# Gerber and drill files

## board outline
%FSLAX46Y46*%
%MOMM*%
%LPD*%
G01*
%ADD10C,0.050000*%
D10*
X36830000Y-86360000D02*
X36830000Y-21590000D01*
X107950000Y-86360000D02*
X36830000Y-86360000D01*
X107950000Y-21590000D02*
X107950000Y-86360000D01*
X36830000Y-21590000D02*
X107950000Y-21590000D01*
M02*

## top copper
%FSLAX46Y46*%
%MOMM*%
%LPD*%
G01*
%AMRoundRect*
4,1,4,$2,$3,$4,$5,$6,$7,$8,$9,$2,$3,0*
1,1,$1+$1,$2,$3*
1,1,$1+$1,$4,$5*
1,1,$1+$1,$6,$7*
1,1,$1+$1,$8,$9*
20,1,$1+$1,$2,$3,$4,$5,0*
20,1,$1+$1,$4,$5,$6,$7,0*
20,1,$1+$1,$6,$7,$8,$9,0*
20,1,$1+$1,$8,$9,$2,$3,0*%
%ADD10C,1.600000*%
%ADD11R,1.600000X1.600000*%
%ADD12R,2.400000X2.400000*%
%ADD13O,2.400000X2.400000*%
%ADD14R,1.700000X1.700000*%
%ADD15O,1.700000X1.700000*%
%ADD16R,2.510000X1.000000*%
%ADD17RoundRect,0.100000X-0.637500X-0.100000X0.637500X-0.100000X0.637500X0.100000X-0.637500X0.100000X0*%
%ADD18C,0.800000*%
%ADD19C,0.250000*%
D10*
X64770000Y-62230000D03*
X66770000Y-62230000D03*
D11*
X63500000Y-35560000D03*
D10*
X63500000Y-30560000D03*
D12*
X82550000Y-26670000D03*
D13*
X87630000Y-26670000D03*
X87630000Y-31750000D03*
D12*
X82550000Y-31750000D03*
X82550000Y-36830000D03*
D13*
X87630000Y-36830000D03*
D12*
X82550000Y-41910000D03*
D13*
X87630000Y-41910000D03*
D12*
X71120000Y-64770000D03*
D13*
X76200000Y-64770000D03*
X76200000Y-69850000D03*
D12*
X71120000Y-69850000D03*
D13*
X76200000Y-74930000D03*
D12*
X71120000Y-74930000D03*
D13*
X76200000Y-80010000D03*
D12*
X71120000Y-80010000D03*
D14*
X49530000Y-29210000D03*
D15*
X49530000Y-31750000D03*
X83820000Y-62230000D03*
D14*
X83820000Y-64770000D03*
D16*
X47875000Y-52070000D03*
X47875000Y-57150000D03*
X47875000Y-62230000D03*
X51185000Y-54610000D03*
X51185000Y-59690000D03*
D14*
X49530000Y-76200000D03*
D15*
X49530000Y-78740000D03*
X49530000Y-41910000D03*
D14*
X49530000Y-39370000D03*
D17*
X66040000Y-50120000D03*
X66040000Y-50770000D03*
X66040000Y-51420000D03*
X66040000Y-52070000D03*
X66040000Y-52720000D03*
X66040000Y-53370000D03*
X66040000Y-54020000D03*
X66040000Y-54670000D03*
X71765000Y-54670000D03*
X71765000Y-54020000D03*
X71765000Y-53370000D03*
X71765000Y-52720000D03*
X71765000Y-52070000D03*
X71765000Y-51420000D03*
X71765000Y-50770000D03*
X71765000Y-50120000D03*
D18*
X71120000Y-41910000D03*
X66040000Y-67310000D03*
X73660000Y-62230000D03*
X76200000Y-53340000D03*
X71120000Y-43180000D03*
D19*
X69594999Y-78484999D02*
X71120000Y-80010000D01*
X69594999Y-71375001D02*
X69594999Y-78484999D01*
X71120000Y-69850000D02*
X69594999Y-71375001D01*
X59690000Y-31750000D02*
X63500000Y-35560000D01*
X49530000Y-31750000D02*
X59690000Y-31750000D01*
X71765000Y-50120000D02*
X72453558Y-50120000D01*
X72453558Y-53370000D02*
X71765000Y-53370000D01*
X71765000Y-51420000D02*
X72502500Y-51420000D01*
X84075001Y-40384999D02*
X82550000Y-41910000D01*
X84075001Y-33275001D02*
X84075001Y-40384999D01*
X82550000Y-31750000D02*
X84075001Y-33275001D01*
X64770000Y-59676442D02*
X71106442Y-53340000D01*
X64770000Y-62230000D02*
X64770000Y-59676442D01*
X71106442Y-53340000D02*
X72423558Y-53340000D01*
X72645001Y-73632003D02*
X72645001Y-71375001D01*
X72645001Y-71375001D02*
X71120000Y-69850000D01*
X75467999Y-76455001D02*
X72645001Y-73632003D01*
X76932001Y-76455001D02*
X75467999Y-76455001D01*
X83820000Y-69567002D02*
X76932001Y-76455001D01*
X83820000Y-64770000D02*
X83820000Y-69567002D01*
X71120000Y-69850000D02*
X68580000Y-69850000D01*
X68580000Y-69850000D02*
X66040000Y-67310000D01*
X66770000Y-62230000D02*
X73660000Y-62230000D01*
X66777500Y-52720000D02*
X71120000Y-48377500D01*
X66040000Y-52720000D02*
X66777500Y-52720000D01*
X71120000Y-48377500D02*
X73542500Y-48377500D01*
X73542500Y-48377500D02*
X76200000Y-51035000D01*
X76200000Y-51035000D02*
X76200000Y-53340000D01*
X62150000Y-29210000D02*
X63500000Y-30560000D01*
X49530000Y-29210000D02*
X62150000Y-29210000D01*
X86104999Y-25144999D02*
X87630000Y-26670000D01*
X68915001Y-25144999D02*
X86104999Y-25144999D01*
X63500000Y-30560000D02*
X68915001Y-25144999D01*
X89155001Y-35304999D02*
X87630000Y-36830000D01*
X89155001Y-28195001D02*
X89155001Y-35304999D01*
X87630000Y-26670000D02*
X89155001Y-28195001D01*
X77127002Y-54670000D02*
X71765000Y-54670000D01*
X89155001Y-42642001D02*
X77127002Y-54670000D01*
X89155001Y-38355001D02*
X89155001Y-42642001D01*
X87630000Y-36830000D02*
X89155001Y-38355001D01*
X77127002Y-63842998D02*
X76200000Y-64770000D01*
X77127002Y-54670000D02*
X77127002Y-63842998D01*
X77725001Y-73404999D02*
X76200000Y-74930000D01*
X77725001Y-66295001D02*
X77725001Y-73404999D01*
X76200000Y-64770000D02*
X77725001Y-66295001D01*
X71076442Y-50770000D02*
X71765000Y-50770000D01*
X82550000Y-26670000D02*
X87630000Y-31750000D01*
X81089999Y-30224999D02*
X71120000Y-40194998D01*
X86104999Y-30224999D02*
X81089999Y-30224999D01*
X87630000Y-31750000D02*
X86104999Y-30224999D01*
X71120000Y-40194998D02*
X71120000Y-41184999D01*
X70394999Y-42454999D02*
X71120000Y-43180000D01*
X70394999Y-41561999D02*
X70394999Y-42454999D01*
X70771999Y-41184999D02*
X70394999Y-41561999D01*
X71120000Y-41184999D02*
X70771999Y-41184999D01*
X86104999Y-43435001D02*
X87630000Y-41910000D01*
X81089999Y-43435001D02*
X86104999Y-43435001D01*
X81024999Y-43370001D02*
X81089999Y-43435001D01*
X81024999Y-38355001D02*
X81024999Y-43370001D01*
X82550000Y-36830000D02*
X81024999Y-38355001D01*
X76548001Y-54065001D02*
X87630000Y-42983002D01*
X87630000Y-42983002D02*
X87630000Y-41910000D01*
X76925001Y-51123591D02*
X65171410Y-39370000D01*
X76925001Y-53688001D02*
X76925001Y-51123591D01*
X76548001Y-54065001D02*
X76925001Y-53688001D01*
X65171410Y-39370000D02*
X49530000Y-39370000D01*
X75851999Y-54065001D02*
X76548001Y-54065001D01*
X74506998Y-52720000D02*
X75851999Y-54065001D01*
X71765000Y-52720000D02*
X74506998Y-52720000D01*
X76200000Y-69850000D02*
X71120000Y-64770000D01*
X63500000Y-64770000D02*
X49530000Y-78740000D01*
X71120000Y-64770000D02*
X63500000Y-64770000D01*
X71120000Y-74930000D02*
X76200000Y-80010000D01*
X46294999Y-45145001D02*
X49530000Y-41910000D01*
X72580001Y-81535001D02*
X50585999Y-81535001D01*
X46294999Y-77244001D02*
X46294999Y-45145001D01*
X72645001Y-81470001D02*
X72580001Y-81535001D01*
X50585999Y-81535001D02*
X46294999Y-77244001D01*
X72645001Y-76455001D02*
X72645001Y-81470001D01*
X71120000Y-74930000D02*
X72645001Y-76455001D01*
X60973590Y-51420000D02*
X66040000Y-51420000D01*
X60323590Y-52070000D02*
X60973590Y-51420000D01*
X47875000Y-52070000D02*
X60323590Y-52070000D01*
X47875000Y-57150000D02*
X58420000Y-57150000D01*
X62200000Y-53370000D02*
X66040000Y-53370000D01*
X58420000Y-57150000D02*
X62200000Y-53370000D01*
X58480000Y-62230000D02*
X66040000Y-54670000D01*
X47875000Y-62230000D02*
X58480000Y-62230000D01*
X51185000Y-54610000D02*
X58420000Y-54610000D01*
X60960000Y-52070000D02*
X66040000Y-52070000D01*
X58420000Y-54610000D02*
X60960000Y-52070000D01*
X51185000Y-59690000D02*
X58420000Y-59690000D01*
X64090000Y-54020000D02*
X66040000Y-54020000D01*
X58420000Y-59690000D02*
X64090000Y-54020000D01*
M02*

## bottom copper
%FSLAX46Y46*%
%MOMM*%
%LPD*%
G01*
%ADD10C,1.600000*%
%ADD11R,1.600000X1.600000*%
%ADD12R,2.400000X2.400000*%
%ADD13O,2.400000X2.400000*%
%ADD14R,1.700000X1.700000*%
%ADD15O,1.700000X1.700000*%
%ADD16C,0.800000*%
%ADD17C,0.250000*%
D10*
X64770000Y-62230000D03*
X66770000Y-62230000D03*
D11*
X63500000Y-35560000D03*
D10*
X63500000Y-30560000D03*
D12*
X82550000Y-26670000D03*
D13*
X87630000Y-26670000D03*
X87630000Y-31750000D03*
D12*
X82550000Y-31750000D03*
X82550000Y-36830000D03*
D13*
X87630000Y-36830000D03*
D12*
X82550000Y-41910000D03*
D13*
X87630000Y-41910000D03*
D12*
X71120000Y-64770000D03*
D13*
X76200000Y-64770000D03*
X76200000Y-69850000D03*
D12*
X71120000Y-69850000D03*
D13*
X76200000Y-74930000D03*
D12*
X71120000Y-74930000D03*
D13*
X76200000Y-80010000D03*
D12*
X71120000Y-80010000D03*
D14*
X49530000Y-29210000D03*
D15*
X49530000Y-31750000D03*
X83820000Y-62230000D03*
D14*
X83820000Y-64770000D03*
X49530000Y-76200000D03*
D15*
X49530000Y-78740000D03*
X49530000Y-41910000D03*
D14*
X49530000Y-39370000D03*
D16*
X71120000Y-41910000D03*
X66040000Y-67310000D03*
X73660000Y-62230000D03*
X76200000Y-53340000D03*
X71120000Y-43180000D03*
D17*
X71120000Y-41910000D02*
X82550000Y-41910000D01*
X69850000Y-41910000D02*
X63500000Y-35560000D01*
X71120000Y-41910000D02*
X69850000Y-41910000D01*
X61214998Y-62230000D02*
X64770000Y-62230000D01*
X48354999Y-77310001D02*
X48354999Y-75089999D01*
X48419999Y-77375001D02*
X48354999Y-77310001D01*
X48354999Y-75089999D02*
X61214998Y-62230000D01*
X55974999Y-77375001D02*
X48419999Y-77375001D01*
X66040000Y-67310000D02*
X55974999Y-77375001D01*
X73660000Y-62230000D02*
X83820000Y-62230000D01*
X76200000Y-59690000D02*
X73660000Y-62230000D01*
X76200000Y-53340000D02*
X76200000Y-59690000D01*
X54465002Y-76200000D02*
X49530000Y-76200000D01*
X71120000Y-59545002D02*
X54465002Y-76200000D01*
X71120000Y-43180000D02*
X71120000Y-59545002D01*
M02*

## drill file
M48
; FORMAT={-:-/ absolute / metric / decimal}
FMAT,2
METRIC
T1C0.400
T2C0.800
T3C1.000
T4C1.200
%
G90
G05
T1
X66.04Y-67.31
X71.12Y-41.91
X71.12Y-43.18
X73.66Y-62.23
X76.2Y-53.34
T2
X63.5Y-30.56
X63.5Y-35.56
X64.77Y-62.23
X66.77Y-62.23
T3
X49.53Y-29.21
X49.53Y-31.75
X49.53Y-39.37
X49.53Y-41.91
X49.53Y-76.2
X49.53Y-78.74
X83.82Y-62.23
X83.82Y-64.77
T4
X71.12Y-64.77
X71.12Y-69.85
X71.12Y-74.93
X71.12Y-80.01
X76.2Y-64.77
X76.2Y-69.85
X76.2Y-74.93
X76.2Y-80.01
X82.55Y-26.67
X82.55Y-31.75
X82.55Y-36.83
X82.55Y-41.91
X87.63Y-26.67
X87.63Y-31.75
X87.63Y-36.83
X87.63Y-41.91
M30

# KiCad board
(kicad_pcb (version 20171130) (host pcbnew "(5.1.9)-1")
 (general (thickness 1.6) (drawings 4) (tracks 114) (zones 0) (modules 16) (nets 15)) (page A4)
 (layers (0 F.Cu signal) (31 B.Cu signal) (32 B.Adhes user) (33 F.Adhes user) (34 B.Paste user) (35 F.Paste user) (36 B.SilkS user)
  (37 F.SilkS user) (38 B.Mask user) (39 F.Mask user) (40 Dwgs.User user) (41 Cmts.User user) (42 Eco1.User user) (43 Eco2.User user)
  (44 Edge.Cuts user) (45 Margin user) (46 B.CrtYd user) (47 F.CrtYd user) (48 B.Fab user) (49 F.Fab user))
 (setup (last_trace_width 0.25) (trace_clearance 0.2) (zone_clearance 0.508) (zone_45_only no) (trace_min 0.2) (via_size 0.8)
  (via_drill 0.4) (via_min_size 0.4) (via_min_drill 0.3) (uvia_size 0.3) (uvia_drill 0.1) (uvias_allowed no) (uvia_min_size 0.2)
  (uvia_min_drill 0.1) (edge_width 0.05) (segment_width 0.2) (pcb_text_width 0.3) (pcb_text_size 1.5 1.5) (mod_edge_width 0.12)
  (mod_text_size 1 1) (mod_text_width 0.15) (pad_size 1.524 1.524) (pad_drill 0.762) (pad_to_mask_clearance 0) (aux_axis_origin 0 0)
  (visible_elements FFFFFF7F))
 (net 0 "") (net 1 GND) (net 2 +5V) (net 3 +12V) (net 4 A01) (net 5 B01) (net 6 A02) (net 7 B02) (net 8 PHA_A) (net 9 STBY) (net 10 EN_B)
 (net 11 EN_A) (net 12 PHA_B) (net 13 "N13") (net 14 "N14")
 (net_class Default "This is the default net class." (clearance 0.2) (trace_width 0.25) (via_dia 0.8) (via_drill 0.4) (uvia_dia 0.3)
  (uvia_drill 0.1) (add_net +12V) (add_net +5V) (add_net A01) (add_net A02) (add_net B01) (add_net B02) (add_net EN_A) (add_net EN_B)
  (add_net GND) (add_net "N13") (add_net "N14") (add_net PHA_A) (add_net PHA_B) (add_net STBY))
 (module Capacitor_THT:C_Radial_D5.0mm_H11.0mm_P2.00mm (layer F.Cu) (at 64.77 62.23)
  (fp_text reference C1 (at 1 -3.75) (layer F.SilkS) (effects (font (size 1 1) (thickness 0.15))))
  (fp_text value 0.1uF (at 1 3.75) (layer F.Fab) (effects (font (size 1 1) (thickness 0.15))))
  (pad 1 thru_hole circle (at 0 0) (size 1.6 1.6) (drill 0.8) (layers *.Cu *.Mask) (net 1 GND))
  (pad 2 thru_hole circle (at 2 0) (size 1.6 1.6) (drill 0.8) (layers *.Cu *.Mask) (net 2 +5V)))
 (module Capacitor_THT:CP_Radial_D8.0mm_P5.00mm (layer F.Cu) (at 63.5 35.56 90)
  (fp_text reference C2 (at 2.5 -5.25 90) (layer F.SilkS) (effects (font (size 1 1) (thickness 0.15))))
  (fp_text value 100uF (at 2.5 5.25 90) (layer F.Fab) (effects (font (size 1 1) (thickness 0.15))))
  (pad 1 thru_hole rect (at 0 0 90) (size 1.6 1.6) (drill 0.8) (layers *.Cu *.Mask) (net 1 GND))
  (pad 2 thru_hole circle (at 5 0 90) (size 1.6 1.6) (drill 0.8) (layers *.Cu *.Mask) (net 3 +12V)))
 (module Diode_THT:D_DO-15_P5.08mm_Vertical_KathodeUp (layer F.Cu) (at 82.55 26.67)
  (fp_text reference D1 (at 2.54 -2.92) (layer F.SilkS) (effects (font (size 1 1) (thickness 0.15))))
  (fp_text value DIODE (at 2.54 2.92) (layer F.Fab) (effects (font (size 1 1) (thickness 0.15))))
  (pad 1 thru_hole rect (at 0 0) (size 2.4 2.4) (drill 1.2) (layers *.Cu *.Mask) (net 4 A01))
  (pad 2 thru_hole oval (at 5.08 0) (size 2.4 2.4) (drill 1.2) (layers *.Cu *.Mask) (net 3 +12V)))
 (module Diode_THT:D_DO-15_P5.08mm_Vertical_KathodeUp (layer F.Cu) (at 82.55 31.75)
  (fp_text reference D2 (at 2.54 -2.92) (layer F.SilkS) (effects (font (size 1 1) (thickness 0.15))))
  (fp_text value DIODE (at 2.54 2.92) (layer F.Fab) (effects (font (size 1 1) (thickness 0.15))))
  (pad 2 thru_hole oval (at 5.08 0) (size 2.4 2.4) (drill 1.2) (layers *.Cu *.Mask) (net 4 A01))
  (pad 1 thru_hole rect (at 0 0) (size 2.4 2.4) (drill 1.2) (layers *.Cu *.Mask) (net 1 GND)))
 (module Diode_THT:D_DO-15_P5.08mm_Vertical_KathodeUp (layer F.Cu) (at 82.55 36.83)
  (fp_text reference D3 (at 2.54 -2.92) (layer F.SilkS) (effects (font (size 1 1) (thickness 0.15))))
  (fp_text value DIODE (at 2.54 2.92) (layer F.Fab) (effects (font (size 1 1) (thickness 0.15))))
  (pad 1 thru_hole rect (at 0 0) (size 2.4 2.4) (drill 1.2) (layers *.Cu *.Mask) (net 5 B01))
  (pad 2 thru_hole oval (at 5.08 0) (size 2.4 2.4) (drill 1.2) (layers *.Cu *.Mask) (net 3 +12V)))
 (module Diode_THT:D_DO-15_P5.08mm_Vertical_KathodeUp (layer F.Cu) (at 82.55 41.91)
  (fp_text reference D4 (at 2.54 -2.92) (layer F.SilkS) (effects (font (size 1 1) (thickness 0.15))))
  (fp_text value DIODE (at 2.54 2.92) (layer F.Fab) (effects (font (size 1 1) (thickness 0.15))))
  (pad 1 thru_hole rect (at 0 0) (size 2.4 2.4) (drill 1.2) (layers *.Cu *.Mask) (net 1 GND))
  (pad 2 thru_hole oval (at 5.08 0) (size 2.4 2.4) (drill 1.2) (layers *.Cu *.Mask) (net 5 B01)))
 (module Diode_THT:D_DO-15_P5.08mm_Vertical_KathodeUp (layer F.Cu) (at 71.12 64.77)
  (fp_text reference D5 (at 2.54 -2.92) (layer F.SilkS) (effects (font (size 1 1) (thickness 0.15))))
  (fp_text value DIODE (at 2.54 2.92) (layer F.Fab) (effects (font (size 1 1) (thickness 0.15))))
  (pad 1 thru_hole rect (at 0 0) (size 2.4 2.4) (drill 1.2) (layers *.Cu *.Mask) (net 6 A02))
  (pad 2 thru_hole oval (at 5.08 0) (size 2.4 2.4) (drill 1.2) (layers *.Cu *.Mask) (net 3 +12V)))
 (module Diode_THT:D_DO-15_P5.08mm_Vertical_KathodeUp (layer F.Cu) (at 71.12 69.85)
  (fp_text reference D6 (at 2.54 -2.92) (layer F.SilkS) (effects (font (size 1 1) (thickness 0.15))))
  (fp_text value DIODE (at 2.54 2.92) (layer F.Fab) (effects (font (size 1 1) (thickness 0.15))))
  (pad 2 thru_hole oval (at 5.08 0) (size 2.4 2.4) (drill 1.2) (layers *.Cu *.Mask) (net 6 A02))
  (pad 1 thru_hole rect (at 0 0) (size 2.4 2.4) (drill 1.2) (layers *.Cu *.Mask) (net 1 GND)))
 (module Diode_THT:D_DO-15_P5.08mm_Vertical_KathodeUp (layer F.Cu) (at 71.12 74.93)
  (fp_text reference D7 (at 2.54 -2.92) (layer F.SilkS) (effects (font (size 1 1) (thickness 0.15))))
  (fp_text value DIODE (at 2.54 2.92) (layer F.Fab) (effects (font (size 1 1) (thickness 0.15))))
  (pad 2 thru_hole oval (at 5.08 0) (size 2.4 2.4) (drill 1.2) (layers *.Cu *.Mask) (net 3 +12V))
  (pad 1 thru_hole rect (at 0 0) (size 2.4 2.4) (drill 1.2) (layers *.Cu *.Mask) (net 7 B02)))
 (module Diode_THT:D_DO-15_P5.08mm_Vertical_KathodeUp (layer F.Cu) (at 71.12 80.01)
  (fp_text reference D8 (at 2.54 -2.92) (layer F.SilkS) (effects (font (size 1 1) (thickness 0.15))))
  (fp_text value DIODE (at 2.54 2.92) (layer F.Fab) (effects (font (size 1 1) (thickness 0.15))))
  (pad 2 thru_hole oval (at 5.08 0) (size 2.4 2.4) (drill 1.2) (layers *.Cu *.Mask) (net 7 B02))
  (pad 1 thru_hole rect (at 0 0) (size 2.4 2.4) (drill 1.2) (layers *.Cu *.Mask) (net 1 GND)))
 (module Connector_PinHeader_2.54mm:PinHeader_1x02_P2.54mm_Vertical (layer F.Cu) (at 49.53 29.21)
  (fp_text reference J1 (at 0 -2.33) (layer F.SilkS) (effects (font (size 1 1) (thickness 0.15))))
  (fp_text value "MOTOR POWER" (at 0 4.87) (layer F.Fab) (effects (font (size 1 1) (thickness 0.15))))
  (pad 1 thru_hole rect (at 0 0) (size 1.7 1.7) (drill 1) (layers *.Cu *.Mask) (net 3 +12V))
  (pad 2 thru_hole oval (at 0 2.54) (size 1.7 1.7) (drill 1) (layers *.Cu *.Mask) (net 1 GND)))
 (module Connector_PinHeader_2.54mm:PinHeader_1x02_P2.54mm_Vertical (layer F.Cu) (at 83.82 64.77 180)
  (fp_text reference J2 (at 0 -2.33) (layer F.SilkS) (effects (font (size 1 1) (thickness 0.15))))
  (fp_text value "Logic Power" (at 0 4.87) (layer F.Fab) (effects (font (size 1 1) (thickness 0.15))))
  (pad 2 thru_hole oval (at 0 2.54 180) (size 1.7 1.7) (drill 1) (layers *.Cu *.Mask) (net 2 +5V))
  (pad 1 thru_hole rect (at 0 0 180) (size 1.7 1.7) (drill 1) (layers *.Cu *.Mask) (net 1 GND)))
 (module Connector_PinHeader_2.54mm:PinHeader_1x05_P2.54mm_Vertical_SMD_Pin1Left (layer F.Cu) (at 49.53 57.15)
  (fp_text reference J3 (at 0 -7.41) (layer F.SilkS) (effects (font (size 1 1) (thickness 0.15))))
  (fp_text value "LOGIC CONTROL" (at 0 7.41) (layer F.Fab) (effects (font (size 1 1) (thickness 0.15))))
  (pad 1 smd rect (at -1.655 -5.08) (size 2.51 1) (layers F.Cu F.Paste F.Mask) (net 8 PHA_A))
  (pad 3 smd rect (at -1.655 0) (size 2.51 1) (layers F.Cu F.Paste F.Mask) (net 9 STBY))
  (pad 5 smd rect (at -1.655 5.08) (size 2.51 1) (layers F.Cu F.Paste F.Mask) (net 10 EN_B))
  (pad 2 smd rect (at 1.655 -2.54) (size 2.51 1) (layers F.Cu F.Paste F.Mask) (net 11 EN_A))
  (pad 4 smd rect (at 1.655 2.54) (size 2.51 1) (layers F.Cu F.Paste F.Mask) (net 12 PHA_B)))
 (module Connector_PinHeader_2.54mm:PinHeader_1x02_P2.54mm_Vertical (layer F.Cu) (at 49.53 76.2)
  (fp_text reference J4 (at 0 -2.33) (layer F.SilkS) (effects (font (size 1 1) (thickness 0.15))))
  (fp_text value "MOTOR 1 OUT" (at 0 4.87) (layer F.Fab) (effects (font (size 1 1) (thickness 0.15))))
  (pad 1 thru_hole rect (at 0 0) (size 1.7 1.7) (drill 1) (layers *.Cu *.Mask) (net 4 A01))
  (pad 2 thru_hole oval (at 0 2.54) (size 1.7 1.7) (drill 1) (layers *.Cu *.Mask) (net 6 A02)))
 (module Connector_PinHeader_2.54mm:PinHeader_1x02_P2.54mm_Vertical (layer F.Cu) (at 49.53 39.37)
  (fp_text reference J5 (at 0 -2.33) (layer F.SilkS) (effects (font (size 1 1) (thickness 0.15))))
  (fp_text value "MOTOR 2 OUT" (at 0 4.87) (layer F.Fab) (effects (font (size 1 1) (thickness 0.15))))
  (pad 2 thru_hole oval (at 0 2.54) (size 1.7 1.7) (drill 1) (layers *.Cu *.Mask) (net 7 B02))
  (pad 1 thru_hole rect (at 0 0) (size 1.7 1.7) (drill 1) (layers *.Cu *.Mask) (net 5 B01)))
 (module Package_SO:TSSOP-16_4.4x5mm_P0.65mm (layer F.Cu) (at 68.9025 52.395)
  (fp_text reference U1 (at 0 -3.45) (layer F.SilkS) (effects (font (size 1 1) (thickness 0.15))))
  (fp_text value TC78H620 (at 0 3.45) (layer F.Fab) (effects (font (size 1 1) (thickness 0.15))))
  (pad 1 smd roundrect (at -2.8625 -2.275) (size 1.475 0.4) (layers F.Cu F.Paste F.Mask) (roundrect_rratio 0.25) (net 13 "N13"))
  (pad 2 smd roundrect (at -2.8625 -1.625) (size 1.475 0.4) (layers F.Cu F.Paste F.Mask) (roundrect_rratio 0.25) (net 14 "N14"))
  (pad 3 smd roundrect (at -2.8625 -0.975) (size 1.475 0.4) (layers F.Cu F.Paste F.Mask) (roundrect_rratio 0.25) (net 8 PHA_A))
  (pad 4 smd roundrect (at -2.8625 -0.325) (size 1.475 0.4) (layers F.Cu F.Paste F.Mask) (roundrect_rratio 0.25) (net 11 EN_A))
  (pad 5 smd roundrect (at -2.8625 0.325) (size 1.475 0.4) (layers F.Cu F.Paste F.Mask) (roundrect_rratio 0.25) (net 2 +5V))
  (pad 6 smd roundrect (at -2.8625 0.975) (size 1.475 0.4) (layers F.Cu F.Paste F.Mask) (roundrect_rratio 0.25) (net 9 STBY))
  (pad 7 smd roundrect (at -2.8625 1.625) (size 1.475 0.4) (layers F.Cu F.Paste F.Mask) (roundrect_rratio 0.25) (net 12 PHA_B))
  (pad 8 smd roundrect (at -2.8625 2.275) (size 1.475 0.4) (layers F.Cu F.Paste F.Mask) (roundrect_rratio 0.25) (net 10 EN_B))
  (pad 9 smd roundrect (at 2.8625 2.275) (size 1.475 0.4) (layers F.Cu F.Paste F.Mask) (roundrect_rratio 0.25) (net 3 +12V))
  (pad 10 smd roundrect (at 2.8625 1.625) (size 1.475 0.4) (layers F.Cu F.Paste F.Mask) (roundrect_rratio 0.25) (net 7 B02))
  (pad 11 smd roundrect (at 2.8625 0.975) (size 1.475 0.4) (layers F.Cu F.Paste F.Mask) (roundrect_rratio 0.25) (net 1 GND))
  (pad 12 smd roundrect (at 2.8625 0.325) (size 1.475 0.4) (layers F.Cu F.Paste F.Mask) (roundrect_rratio 0.25) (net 5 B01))
  (pad 13 smd roundrect (at 2.8625 -0.325) (size 1.475 0.4) (layers F.Cu F.Paste F.Mask) (roundrect_rratio 0.25) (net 6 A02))
  (pad 14 smd roundrect (at 2.8625 -0.975) (size 1.475 0.4) (layers F.Cu F.Paste F.Mask) (roundrect_rratio 0.25) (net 1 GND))
  (pad 15 smd roundrect (at 2.8625 -1.625) (size 1.475 0.4) (layers F.Cu F.Paste F.Mask) (roundrect_rratio 0.25) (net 4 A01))
  (pad 16 smd roundrect (at 2.8625 -2.275) (size 1.475 0.4) (layers F.Cu F.Paste F.Mask) (roundrect_rratio 0.25) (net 1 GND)))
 (gr_line (start 36.83 86.36) (end 36.83 21.59) (layer Edge.Cuts) (width 0.05))
 (gr_line (start 107.95 86.36) (end 36.83 86.36) (layer Edge.Cuts) (width 0.05))
 (gr_line (start 107.95 21.59) (end 107.95 86.36) (layer Edge.Cuts) (width 0.05))
 (gr_line (start 36.83 21.59) (end 107.95 21.59) (layer Edge.Cuts) (width 0.05))
 (segment (start 69.594999 78.484999) (end 71.12 80.01) (width 0.25) (layer F.Cu) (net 1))
 (segment (start 69.594999 71.375001) (end 69.594999 78.484999) (width 0.25) (layer F.Cu) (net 1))
 (segment (start 71.12 69.85) (end 69.594999 71.375001) (width 0.25) (layer F.Cu) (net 1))
 (segment (start 59.69 31.75) (end 63.5 35.56) (width 0.25) (layer F.Cu) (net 1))
 (segment (start 49.53 31.75) (end 59.69 31.75) (width 0.25) (layer F.Cu) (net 1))
 (segment (start 71.765 50.12) (end 72.453558 50.12) (width 0.25) (layer F.Cu) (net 1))
 (segment (start 72.453558 53.37) (end 71.765 53.37) (width 0.25) (layer F.Cu) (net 1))
 (segment (start 71.765 51.42) (end 72.5025 51.42) (width 0.25) (layer F.Cu) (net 1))
 (via (at 71.12 41.91) (size 0.8) (drill 0.4) (layers F.Cu B.Cu) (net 1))
 (segment (start 71.12 41.91) (end 82.55 41.91) (width 0.25) (layer B.Cu) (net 1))
 (segment (start 69.85 41.91) (end 63.5 35.56) (width 0.25) (layer B.Cu) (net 1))
 (segment (start 71.12 41.91) (end 69.85 41.91) (width 0.25) (layer B.Cu) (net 1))
 (segment (start 84.075001 40.384999) (end 82.55 41.91) (width 0.25) (layer F.Cu) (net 1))
 (segment (start 84.075001 33.275001) (end 84.075001 40.384999) (width 0.25) (layer F.Cu) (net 1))
 (segment (start 82.55 31.75) (end 84.075001 33.275001) (width 0.25) (layer F.Cu) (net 1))
 (segment (start 64.77 59.676442) (end 71.106442 53.34) (width 0.25) (layer F.Cu) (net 1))
 (segment (start 64.77 62.23) (end 64.77 59.676442) (width 0.25) (layer F.Cu) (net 1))
 (segment (start 71.106442 53.34) (end 72.423558 53.34) (width 0.25) (layer F.Cu) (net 1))
 (segment (start 72.645001 73.632003) (end 72.645001 71.375001) (width 0.25) (layer F.Cu) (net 1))
 (segment (start 72.645001 71.375001) (end 71.12 69.85) (width 0.25) (layer F.Cu) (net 1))
 (segment (start 75.467999 76.455001) (end 72.645001 73.632003) (width 0.25) (layer F.Cu) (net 1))
 (segment (start 76.932001 76.455001) (end 75.467999 76.455001) (width 0.25) (layer F.Cu) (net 1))
 (segment (start 83.82 69.567002) (end 76.932001 76.455001) (width 0.25) (layer F.Cu) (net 1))
 (segment (start 83.82 64.77) (end 83.82 69.567002) (width 0.25) (layer F.Cu) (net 1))
 (segment (start 71.12 69.85) (end 68.58 69.85) (width 0.25) (layer F.Cu) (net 1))
 (via (at 66.04 67.31) (size 0.8) (drill 0.4) (layers F.Cu B.Cu) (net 1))
 (segment (start 68.58 69.85) (end 66.04 67.31) (width 0.25) (layer F.Cu) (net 1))
 (segment (start 61.214998 62.23) (end 64.77 62.23) (width 0.25) (layer B.Cu) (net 1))
 (segment (start 48.354999 77.310001) (end 48.354999 75.089999) (width 0.25) (layer B.Cu) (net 1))
 (segment (start 48.419999 77.375001) (end 48.354999 77.310001) (width 0.25) (layer B.Cu) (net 1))
 (segment (start 48.354999 75.089999) (end 61.214998 62.23) (width 0.25) (layer B.Cu) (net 1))
 (segment (start 55.974999 77.375001) (end 48.419999 77.375001) (width 0.25) (layer B.Cu) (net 1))
 (segment (start 66.04 67.31) (end 55.974999 77.375001) (width 0.25) (layer B.Cu) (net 1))
 (via (at 73.66 62.23) (size 0.8) (drill 0.4) (layers F.Cu B.Cu) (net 2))
 (segment (start 66.77 62.23) (end 73.66 62.23) (width 0.25) (layer F.Cu) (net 2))
 (segment (start 73.66 62.23) (end 83.82 62.23) (width 0.25) (layer B.Cu) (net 2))
 (segment (start 66.7775 52.72) (end 71.12 48.3775) (width 0.25) (layer F.Cu) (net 2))
 (segment (start 66.04 52.72) (end 66.7775 52.72) (width 0.25) (layer F.Cu) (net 2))
 (segment (start 71.12 48.3775) (end 73.5425 48.3775) (width 0.25) (layer F.Cu) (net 2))
 (segment (start 73.5425 48.3775) (end 76.2 51.035) (width 0.25) (layer F.Cu) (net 2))
 (via (at 76.2 53.34) (size 0.8) (drill 0.4) (layers F.Cu B.Cu) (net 2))
 (segment (start 76.2 51.035) (end 76.2 53.34) (width 0.25) (layer F.Cu) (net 2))
 (segment (start 76.2 59.69) (end 73.66 62.23) (width 0.25) (layer B.Cu) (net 2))
 (segment (start 76.2 53.34) (end 76.2 59.69) (width 0.25) (layer B.Cu) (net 2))
 (segment (start 62.15 29.21) (end 63.5 30.56) (width 0.25) (layer F.Cu) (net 3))
 (segment (start 49.53 29.21) (end 62.15 29.21) (width 0.25) (layer F.Cu) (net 3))
 (segment (start 86.104999 25.144999) (end 87.63 26.67) (width 0.25) (layer F.Cu) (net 3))
 (segment (start 68.915001 25.144999) (end 86.104999 25.144999) (width 0.25) (layer F.Cu) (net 3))
 (segment (start 63.5 30.56) (end 68.915001 25.144999) (width 0.25) (layer F.Cu) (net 3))
 (segment (start 89.155001 35.304999) (end 87.63 36.83) (width 0.25) (layer F.Cu) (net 3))
 (segment (start 89.155001 28.195001) (end 89.155001 35.304999) (width 0.25) (layer F.Cu) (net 3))
 (segment (start 87.63 26.67) (end 89.155001 28.195001) (width 0.25) (layer F.Cu) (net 3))
 (segment (start 77.127002 54.67) (end 71.765 54.67) (width 0.25) (layer F.Cu) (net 3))
 (segment (start 89.155001 42.642001) (end 77.127002 54.67) (width 0.25) (layer F.Cu) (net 3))
 (segment (start 89.155001 38.355001) (end 89.155001 42.642001) (width 0.25) (layer F.Cu) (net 3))
 (segment (start 87.63 36.83) (end 89.155001 38.355001) (width 0.25) (layer F.Cu) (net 3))
 (segment (start 77.127002 63.842998) (end 76.2 64.77) (width 0.25) (layer F.Cu) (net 3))
 (segment (start 77.127002 54.67) (end 77.127002 63.842998) (width 0.25) (layer F.Cu) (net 3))
 (segment (start 77.725001 73.404999) (end 76.2 74.93) (width 0.25) (layer F.Cu) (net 3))
 (segment (start 77.725001 66.295001) (end 77.725001 73.404999) (width 0.25) (layer F.Cu) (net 3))
 (segment (start 76.2 64.77) (end 77.725001 66.295001) (width 0.25) (layer F.Cu) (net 3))
 (segment (start 71.076442 50.77) (end 71.765 50.77) (width 0.25) (layer F.Cu) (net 4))
 (segment (start 82.55 26.67) (end 87.63 31.75) (width 0.25) (layer F.Cu) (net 4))
 (segment (start 81.089999 30.224999) (end 71.12 40.194998) (width 0.25) (layer F.Cu) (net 4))
 (segment (start 86.104999 30.224999) (end 81.089999 30.224999) (width 0.25) (layer F.Cu) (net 4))
 (segment (start 87.63 31.75) (end 86.104999 30.224999) (width 0.25) (layer F.Cu) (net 4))
 (segment (start 71.12 40.194998) (end 71.12 41.184999) (width 0.25) (layer F.Cu) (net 4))
 (via (at 71.12 43.18) (size 0.8) (drill 0.4) (layers F.Cu B.Cu) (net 4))
 (segment (start 70.394999 42.454999) (end 71.12 43.18) (width 0.25) (layer F.Cu) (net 4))
 (segment (start 70.394999 41.561999) (end 70.394999 42.454999) (width 0.25) (layer F.Cu) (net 4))
 (segment (start 70.771999 41.184999) (end 70.394999 41.561999) (width 0.25) (layer F.Cu) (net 4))
 (segment (start 71.12 41.184999) (end 70.771999 41.184999) (width 0.25) (layer F.Cu) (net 4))
 (segment (start 54.465002 76.2) (end 49.53 76.2) (width 0.25) (layer B.Cu) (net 4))
 (segment (start 71.12 59.545002) (end 54.465002 76.2) (width 0.25) (layer B.Cu) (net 4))
 (segment (start 71.12 43.18) (end 71.12 59.545002) (width 0.25) (layer B.Cu) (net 4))
 (segment (start 86.104999 43.435001) (end 87.63 41.91) (width 0.25) (layer F.Cu) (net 5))
 (segment (start 81.089999 43.435001) (end 86.104999 43.435001) (width 0.25) (layer F.Cu) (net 5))
 (segment (start 81.024999 43.370001) (end 81.089999 43.435001) (width 0.25) (layer F.Cu) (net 5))
 (segment (start 81.024999 38.355001) (end 81.024999 43.370001) (width 0.25) (layer F.Cu) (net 5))
 (segment (start 82.55 36.83) (end 81.024999 38.355001) (width 0.25) (layer F.Cu) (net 5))
 (segment (start 76.548001 54.065001) (end 87.63 42.983002) (width 0.25) (layer F.Cu) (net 5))
 (segment (start 87.63 42.983002) (end 87.63 41.91) (width 0.25) (layer F.Cu) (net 5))
 (segment (start 76.925001 51.123591) (end 65.17141 39.37) (width 0.25) (layer F.Cu) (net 5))
 (segment (start 76.925001 53.688001) (end 76.925001 51.123591) (width 0.25) (layer F.Cu) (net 5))
 (segment (start 76.548001 54.065001) (end 76.925001 53.688001) (width 0.25) (layer F.Cu) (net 5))
 (segment (start 65.17141 39.37) (end 49.53 39.37) (width 0.25) (layer F.Cu) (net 5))
 (segment (start 75.851999 54.065001) (end 76.548001 54.065001) (width 0.25) (layer F.Cu) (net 5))
 (segment (start 74.506998 52.72) (end 75.851999 54.065001) (width 0.25) (layer F.Cu) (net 5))
 (segment (start 71.765 52.72) (end 74.506998 52.72) (width 0.25) (layer F.Cu) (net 5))
 (segment (start 76.2 69.85) (end 71.12 64.77) (width 0.25) (layer F.Cu) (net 6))
 (segment (start 63.5 64.77) (end 49.53 78.74) (width 0.25) (layer F.Cu) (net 6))
 (segment (start 71.12 64.77) (end 63.5 64.77) (width 0.25) (layer F.Cu) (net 6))
 (segment (start 71.12 74.93) (end 76.2 80.01) (width 0.25) (layer F.Cu) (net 7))
 (segment (start 46.294999 45.145001) (end 49.53 41.91) (width 0.25) (layer F.Cu) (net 7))
 (segment (start 72.580001 81.535001) (end 50.585999 81.535001) (width 0.25) (layer F.Cu) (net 7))
 (segment (start 46.294999 77.244001) (end 46.294999 45.145001) (width 0.25) (layer F.Cu) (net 7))
 (segment (start 72.645001 81.470001) (end 72.580001 81.535001) (width 0.25) (layer F.Cu) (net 7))
 (segment (start 50.585999 81.535001) (end 46.294999 77.244001) (width 0.25) (layer F.Cu) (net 7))
 (segment (start 72.645001 76.455001) (end 72.645001 81.470001) (width 0.25) (layer F.Cu) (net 7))
 (segment (start 71.12 74.93) (end 72.645001 76.455001) (width 0.25) (layer F.Cu) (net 7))
 (segment (start 60.97359 51.42) (end 66.04 51.42) (width 0.25) (layer F.Cu) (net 8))
 (segment (start 60.32359 52.07) (end 60.97359 51.42) (width 0.25) (layer F.Cu) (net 8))
 (segment (start 47.875 52.07) (end 60.32359 52.07) (width 0.25) (layer F.Cu) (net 8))
 (segment (start 47.875 57.15) (end 58.42 57.15) (width 0.25) (layer F.Cu) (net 9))
 (segment (start 62.2 53.37) (end 66.04 53.37) (width 0.25) (layer F.Cu) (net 9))
 (segment (start 58.42 57.15) (end 62.2 53.37) (width 0.25) (layer F.Cu) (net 9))
 (segment (start 58.48 62.23) (end 66.04 54.67) (width 0.25) (layer F.Cu) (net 10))
 (segment (start 47.875 62.23) (end 58.48 62.23) (width 0.25) (layer F.Cu) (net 10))
 (segment (start 51.185 54.61) (end 58.42 54.61) (width 0.25) (layer F.Cu) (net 11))
 (segment (start 60.96 52.07) (end 66.04 52.07) (width 0.25) (layer F.Cu) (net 11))
 (segment (start 58.42 54.61) (end 60.96 52.07) (width 0.25) (layer F.Cu) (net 11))
 (segment (start 51.185 59.69) (end 58.42 59.69) (width 0.25) (layer F.Cu) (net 12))
 (segment (start 64.09 54.02) (end 66.04 54.02) (width 0.25) (layer F.Cu) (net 12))
 (segment (start 58.42 59.69) (end 64.09 54.02) (width 0.25) (layer F.Cu) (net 12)))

